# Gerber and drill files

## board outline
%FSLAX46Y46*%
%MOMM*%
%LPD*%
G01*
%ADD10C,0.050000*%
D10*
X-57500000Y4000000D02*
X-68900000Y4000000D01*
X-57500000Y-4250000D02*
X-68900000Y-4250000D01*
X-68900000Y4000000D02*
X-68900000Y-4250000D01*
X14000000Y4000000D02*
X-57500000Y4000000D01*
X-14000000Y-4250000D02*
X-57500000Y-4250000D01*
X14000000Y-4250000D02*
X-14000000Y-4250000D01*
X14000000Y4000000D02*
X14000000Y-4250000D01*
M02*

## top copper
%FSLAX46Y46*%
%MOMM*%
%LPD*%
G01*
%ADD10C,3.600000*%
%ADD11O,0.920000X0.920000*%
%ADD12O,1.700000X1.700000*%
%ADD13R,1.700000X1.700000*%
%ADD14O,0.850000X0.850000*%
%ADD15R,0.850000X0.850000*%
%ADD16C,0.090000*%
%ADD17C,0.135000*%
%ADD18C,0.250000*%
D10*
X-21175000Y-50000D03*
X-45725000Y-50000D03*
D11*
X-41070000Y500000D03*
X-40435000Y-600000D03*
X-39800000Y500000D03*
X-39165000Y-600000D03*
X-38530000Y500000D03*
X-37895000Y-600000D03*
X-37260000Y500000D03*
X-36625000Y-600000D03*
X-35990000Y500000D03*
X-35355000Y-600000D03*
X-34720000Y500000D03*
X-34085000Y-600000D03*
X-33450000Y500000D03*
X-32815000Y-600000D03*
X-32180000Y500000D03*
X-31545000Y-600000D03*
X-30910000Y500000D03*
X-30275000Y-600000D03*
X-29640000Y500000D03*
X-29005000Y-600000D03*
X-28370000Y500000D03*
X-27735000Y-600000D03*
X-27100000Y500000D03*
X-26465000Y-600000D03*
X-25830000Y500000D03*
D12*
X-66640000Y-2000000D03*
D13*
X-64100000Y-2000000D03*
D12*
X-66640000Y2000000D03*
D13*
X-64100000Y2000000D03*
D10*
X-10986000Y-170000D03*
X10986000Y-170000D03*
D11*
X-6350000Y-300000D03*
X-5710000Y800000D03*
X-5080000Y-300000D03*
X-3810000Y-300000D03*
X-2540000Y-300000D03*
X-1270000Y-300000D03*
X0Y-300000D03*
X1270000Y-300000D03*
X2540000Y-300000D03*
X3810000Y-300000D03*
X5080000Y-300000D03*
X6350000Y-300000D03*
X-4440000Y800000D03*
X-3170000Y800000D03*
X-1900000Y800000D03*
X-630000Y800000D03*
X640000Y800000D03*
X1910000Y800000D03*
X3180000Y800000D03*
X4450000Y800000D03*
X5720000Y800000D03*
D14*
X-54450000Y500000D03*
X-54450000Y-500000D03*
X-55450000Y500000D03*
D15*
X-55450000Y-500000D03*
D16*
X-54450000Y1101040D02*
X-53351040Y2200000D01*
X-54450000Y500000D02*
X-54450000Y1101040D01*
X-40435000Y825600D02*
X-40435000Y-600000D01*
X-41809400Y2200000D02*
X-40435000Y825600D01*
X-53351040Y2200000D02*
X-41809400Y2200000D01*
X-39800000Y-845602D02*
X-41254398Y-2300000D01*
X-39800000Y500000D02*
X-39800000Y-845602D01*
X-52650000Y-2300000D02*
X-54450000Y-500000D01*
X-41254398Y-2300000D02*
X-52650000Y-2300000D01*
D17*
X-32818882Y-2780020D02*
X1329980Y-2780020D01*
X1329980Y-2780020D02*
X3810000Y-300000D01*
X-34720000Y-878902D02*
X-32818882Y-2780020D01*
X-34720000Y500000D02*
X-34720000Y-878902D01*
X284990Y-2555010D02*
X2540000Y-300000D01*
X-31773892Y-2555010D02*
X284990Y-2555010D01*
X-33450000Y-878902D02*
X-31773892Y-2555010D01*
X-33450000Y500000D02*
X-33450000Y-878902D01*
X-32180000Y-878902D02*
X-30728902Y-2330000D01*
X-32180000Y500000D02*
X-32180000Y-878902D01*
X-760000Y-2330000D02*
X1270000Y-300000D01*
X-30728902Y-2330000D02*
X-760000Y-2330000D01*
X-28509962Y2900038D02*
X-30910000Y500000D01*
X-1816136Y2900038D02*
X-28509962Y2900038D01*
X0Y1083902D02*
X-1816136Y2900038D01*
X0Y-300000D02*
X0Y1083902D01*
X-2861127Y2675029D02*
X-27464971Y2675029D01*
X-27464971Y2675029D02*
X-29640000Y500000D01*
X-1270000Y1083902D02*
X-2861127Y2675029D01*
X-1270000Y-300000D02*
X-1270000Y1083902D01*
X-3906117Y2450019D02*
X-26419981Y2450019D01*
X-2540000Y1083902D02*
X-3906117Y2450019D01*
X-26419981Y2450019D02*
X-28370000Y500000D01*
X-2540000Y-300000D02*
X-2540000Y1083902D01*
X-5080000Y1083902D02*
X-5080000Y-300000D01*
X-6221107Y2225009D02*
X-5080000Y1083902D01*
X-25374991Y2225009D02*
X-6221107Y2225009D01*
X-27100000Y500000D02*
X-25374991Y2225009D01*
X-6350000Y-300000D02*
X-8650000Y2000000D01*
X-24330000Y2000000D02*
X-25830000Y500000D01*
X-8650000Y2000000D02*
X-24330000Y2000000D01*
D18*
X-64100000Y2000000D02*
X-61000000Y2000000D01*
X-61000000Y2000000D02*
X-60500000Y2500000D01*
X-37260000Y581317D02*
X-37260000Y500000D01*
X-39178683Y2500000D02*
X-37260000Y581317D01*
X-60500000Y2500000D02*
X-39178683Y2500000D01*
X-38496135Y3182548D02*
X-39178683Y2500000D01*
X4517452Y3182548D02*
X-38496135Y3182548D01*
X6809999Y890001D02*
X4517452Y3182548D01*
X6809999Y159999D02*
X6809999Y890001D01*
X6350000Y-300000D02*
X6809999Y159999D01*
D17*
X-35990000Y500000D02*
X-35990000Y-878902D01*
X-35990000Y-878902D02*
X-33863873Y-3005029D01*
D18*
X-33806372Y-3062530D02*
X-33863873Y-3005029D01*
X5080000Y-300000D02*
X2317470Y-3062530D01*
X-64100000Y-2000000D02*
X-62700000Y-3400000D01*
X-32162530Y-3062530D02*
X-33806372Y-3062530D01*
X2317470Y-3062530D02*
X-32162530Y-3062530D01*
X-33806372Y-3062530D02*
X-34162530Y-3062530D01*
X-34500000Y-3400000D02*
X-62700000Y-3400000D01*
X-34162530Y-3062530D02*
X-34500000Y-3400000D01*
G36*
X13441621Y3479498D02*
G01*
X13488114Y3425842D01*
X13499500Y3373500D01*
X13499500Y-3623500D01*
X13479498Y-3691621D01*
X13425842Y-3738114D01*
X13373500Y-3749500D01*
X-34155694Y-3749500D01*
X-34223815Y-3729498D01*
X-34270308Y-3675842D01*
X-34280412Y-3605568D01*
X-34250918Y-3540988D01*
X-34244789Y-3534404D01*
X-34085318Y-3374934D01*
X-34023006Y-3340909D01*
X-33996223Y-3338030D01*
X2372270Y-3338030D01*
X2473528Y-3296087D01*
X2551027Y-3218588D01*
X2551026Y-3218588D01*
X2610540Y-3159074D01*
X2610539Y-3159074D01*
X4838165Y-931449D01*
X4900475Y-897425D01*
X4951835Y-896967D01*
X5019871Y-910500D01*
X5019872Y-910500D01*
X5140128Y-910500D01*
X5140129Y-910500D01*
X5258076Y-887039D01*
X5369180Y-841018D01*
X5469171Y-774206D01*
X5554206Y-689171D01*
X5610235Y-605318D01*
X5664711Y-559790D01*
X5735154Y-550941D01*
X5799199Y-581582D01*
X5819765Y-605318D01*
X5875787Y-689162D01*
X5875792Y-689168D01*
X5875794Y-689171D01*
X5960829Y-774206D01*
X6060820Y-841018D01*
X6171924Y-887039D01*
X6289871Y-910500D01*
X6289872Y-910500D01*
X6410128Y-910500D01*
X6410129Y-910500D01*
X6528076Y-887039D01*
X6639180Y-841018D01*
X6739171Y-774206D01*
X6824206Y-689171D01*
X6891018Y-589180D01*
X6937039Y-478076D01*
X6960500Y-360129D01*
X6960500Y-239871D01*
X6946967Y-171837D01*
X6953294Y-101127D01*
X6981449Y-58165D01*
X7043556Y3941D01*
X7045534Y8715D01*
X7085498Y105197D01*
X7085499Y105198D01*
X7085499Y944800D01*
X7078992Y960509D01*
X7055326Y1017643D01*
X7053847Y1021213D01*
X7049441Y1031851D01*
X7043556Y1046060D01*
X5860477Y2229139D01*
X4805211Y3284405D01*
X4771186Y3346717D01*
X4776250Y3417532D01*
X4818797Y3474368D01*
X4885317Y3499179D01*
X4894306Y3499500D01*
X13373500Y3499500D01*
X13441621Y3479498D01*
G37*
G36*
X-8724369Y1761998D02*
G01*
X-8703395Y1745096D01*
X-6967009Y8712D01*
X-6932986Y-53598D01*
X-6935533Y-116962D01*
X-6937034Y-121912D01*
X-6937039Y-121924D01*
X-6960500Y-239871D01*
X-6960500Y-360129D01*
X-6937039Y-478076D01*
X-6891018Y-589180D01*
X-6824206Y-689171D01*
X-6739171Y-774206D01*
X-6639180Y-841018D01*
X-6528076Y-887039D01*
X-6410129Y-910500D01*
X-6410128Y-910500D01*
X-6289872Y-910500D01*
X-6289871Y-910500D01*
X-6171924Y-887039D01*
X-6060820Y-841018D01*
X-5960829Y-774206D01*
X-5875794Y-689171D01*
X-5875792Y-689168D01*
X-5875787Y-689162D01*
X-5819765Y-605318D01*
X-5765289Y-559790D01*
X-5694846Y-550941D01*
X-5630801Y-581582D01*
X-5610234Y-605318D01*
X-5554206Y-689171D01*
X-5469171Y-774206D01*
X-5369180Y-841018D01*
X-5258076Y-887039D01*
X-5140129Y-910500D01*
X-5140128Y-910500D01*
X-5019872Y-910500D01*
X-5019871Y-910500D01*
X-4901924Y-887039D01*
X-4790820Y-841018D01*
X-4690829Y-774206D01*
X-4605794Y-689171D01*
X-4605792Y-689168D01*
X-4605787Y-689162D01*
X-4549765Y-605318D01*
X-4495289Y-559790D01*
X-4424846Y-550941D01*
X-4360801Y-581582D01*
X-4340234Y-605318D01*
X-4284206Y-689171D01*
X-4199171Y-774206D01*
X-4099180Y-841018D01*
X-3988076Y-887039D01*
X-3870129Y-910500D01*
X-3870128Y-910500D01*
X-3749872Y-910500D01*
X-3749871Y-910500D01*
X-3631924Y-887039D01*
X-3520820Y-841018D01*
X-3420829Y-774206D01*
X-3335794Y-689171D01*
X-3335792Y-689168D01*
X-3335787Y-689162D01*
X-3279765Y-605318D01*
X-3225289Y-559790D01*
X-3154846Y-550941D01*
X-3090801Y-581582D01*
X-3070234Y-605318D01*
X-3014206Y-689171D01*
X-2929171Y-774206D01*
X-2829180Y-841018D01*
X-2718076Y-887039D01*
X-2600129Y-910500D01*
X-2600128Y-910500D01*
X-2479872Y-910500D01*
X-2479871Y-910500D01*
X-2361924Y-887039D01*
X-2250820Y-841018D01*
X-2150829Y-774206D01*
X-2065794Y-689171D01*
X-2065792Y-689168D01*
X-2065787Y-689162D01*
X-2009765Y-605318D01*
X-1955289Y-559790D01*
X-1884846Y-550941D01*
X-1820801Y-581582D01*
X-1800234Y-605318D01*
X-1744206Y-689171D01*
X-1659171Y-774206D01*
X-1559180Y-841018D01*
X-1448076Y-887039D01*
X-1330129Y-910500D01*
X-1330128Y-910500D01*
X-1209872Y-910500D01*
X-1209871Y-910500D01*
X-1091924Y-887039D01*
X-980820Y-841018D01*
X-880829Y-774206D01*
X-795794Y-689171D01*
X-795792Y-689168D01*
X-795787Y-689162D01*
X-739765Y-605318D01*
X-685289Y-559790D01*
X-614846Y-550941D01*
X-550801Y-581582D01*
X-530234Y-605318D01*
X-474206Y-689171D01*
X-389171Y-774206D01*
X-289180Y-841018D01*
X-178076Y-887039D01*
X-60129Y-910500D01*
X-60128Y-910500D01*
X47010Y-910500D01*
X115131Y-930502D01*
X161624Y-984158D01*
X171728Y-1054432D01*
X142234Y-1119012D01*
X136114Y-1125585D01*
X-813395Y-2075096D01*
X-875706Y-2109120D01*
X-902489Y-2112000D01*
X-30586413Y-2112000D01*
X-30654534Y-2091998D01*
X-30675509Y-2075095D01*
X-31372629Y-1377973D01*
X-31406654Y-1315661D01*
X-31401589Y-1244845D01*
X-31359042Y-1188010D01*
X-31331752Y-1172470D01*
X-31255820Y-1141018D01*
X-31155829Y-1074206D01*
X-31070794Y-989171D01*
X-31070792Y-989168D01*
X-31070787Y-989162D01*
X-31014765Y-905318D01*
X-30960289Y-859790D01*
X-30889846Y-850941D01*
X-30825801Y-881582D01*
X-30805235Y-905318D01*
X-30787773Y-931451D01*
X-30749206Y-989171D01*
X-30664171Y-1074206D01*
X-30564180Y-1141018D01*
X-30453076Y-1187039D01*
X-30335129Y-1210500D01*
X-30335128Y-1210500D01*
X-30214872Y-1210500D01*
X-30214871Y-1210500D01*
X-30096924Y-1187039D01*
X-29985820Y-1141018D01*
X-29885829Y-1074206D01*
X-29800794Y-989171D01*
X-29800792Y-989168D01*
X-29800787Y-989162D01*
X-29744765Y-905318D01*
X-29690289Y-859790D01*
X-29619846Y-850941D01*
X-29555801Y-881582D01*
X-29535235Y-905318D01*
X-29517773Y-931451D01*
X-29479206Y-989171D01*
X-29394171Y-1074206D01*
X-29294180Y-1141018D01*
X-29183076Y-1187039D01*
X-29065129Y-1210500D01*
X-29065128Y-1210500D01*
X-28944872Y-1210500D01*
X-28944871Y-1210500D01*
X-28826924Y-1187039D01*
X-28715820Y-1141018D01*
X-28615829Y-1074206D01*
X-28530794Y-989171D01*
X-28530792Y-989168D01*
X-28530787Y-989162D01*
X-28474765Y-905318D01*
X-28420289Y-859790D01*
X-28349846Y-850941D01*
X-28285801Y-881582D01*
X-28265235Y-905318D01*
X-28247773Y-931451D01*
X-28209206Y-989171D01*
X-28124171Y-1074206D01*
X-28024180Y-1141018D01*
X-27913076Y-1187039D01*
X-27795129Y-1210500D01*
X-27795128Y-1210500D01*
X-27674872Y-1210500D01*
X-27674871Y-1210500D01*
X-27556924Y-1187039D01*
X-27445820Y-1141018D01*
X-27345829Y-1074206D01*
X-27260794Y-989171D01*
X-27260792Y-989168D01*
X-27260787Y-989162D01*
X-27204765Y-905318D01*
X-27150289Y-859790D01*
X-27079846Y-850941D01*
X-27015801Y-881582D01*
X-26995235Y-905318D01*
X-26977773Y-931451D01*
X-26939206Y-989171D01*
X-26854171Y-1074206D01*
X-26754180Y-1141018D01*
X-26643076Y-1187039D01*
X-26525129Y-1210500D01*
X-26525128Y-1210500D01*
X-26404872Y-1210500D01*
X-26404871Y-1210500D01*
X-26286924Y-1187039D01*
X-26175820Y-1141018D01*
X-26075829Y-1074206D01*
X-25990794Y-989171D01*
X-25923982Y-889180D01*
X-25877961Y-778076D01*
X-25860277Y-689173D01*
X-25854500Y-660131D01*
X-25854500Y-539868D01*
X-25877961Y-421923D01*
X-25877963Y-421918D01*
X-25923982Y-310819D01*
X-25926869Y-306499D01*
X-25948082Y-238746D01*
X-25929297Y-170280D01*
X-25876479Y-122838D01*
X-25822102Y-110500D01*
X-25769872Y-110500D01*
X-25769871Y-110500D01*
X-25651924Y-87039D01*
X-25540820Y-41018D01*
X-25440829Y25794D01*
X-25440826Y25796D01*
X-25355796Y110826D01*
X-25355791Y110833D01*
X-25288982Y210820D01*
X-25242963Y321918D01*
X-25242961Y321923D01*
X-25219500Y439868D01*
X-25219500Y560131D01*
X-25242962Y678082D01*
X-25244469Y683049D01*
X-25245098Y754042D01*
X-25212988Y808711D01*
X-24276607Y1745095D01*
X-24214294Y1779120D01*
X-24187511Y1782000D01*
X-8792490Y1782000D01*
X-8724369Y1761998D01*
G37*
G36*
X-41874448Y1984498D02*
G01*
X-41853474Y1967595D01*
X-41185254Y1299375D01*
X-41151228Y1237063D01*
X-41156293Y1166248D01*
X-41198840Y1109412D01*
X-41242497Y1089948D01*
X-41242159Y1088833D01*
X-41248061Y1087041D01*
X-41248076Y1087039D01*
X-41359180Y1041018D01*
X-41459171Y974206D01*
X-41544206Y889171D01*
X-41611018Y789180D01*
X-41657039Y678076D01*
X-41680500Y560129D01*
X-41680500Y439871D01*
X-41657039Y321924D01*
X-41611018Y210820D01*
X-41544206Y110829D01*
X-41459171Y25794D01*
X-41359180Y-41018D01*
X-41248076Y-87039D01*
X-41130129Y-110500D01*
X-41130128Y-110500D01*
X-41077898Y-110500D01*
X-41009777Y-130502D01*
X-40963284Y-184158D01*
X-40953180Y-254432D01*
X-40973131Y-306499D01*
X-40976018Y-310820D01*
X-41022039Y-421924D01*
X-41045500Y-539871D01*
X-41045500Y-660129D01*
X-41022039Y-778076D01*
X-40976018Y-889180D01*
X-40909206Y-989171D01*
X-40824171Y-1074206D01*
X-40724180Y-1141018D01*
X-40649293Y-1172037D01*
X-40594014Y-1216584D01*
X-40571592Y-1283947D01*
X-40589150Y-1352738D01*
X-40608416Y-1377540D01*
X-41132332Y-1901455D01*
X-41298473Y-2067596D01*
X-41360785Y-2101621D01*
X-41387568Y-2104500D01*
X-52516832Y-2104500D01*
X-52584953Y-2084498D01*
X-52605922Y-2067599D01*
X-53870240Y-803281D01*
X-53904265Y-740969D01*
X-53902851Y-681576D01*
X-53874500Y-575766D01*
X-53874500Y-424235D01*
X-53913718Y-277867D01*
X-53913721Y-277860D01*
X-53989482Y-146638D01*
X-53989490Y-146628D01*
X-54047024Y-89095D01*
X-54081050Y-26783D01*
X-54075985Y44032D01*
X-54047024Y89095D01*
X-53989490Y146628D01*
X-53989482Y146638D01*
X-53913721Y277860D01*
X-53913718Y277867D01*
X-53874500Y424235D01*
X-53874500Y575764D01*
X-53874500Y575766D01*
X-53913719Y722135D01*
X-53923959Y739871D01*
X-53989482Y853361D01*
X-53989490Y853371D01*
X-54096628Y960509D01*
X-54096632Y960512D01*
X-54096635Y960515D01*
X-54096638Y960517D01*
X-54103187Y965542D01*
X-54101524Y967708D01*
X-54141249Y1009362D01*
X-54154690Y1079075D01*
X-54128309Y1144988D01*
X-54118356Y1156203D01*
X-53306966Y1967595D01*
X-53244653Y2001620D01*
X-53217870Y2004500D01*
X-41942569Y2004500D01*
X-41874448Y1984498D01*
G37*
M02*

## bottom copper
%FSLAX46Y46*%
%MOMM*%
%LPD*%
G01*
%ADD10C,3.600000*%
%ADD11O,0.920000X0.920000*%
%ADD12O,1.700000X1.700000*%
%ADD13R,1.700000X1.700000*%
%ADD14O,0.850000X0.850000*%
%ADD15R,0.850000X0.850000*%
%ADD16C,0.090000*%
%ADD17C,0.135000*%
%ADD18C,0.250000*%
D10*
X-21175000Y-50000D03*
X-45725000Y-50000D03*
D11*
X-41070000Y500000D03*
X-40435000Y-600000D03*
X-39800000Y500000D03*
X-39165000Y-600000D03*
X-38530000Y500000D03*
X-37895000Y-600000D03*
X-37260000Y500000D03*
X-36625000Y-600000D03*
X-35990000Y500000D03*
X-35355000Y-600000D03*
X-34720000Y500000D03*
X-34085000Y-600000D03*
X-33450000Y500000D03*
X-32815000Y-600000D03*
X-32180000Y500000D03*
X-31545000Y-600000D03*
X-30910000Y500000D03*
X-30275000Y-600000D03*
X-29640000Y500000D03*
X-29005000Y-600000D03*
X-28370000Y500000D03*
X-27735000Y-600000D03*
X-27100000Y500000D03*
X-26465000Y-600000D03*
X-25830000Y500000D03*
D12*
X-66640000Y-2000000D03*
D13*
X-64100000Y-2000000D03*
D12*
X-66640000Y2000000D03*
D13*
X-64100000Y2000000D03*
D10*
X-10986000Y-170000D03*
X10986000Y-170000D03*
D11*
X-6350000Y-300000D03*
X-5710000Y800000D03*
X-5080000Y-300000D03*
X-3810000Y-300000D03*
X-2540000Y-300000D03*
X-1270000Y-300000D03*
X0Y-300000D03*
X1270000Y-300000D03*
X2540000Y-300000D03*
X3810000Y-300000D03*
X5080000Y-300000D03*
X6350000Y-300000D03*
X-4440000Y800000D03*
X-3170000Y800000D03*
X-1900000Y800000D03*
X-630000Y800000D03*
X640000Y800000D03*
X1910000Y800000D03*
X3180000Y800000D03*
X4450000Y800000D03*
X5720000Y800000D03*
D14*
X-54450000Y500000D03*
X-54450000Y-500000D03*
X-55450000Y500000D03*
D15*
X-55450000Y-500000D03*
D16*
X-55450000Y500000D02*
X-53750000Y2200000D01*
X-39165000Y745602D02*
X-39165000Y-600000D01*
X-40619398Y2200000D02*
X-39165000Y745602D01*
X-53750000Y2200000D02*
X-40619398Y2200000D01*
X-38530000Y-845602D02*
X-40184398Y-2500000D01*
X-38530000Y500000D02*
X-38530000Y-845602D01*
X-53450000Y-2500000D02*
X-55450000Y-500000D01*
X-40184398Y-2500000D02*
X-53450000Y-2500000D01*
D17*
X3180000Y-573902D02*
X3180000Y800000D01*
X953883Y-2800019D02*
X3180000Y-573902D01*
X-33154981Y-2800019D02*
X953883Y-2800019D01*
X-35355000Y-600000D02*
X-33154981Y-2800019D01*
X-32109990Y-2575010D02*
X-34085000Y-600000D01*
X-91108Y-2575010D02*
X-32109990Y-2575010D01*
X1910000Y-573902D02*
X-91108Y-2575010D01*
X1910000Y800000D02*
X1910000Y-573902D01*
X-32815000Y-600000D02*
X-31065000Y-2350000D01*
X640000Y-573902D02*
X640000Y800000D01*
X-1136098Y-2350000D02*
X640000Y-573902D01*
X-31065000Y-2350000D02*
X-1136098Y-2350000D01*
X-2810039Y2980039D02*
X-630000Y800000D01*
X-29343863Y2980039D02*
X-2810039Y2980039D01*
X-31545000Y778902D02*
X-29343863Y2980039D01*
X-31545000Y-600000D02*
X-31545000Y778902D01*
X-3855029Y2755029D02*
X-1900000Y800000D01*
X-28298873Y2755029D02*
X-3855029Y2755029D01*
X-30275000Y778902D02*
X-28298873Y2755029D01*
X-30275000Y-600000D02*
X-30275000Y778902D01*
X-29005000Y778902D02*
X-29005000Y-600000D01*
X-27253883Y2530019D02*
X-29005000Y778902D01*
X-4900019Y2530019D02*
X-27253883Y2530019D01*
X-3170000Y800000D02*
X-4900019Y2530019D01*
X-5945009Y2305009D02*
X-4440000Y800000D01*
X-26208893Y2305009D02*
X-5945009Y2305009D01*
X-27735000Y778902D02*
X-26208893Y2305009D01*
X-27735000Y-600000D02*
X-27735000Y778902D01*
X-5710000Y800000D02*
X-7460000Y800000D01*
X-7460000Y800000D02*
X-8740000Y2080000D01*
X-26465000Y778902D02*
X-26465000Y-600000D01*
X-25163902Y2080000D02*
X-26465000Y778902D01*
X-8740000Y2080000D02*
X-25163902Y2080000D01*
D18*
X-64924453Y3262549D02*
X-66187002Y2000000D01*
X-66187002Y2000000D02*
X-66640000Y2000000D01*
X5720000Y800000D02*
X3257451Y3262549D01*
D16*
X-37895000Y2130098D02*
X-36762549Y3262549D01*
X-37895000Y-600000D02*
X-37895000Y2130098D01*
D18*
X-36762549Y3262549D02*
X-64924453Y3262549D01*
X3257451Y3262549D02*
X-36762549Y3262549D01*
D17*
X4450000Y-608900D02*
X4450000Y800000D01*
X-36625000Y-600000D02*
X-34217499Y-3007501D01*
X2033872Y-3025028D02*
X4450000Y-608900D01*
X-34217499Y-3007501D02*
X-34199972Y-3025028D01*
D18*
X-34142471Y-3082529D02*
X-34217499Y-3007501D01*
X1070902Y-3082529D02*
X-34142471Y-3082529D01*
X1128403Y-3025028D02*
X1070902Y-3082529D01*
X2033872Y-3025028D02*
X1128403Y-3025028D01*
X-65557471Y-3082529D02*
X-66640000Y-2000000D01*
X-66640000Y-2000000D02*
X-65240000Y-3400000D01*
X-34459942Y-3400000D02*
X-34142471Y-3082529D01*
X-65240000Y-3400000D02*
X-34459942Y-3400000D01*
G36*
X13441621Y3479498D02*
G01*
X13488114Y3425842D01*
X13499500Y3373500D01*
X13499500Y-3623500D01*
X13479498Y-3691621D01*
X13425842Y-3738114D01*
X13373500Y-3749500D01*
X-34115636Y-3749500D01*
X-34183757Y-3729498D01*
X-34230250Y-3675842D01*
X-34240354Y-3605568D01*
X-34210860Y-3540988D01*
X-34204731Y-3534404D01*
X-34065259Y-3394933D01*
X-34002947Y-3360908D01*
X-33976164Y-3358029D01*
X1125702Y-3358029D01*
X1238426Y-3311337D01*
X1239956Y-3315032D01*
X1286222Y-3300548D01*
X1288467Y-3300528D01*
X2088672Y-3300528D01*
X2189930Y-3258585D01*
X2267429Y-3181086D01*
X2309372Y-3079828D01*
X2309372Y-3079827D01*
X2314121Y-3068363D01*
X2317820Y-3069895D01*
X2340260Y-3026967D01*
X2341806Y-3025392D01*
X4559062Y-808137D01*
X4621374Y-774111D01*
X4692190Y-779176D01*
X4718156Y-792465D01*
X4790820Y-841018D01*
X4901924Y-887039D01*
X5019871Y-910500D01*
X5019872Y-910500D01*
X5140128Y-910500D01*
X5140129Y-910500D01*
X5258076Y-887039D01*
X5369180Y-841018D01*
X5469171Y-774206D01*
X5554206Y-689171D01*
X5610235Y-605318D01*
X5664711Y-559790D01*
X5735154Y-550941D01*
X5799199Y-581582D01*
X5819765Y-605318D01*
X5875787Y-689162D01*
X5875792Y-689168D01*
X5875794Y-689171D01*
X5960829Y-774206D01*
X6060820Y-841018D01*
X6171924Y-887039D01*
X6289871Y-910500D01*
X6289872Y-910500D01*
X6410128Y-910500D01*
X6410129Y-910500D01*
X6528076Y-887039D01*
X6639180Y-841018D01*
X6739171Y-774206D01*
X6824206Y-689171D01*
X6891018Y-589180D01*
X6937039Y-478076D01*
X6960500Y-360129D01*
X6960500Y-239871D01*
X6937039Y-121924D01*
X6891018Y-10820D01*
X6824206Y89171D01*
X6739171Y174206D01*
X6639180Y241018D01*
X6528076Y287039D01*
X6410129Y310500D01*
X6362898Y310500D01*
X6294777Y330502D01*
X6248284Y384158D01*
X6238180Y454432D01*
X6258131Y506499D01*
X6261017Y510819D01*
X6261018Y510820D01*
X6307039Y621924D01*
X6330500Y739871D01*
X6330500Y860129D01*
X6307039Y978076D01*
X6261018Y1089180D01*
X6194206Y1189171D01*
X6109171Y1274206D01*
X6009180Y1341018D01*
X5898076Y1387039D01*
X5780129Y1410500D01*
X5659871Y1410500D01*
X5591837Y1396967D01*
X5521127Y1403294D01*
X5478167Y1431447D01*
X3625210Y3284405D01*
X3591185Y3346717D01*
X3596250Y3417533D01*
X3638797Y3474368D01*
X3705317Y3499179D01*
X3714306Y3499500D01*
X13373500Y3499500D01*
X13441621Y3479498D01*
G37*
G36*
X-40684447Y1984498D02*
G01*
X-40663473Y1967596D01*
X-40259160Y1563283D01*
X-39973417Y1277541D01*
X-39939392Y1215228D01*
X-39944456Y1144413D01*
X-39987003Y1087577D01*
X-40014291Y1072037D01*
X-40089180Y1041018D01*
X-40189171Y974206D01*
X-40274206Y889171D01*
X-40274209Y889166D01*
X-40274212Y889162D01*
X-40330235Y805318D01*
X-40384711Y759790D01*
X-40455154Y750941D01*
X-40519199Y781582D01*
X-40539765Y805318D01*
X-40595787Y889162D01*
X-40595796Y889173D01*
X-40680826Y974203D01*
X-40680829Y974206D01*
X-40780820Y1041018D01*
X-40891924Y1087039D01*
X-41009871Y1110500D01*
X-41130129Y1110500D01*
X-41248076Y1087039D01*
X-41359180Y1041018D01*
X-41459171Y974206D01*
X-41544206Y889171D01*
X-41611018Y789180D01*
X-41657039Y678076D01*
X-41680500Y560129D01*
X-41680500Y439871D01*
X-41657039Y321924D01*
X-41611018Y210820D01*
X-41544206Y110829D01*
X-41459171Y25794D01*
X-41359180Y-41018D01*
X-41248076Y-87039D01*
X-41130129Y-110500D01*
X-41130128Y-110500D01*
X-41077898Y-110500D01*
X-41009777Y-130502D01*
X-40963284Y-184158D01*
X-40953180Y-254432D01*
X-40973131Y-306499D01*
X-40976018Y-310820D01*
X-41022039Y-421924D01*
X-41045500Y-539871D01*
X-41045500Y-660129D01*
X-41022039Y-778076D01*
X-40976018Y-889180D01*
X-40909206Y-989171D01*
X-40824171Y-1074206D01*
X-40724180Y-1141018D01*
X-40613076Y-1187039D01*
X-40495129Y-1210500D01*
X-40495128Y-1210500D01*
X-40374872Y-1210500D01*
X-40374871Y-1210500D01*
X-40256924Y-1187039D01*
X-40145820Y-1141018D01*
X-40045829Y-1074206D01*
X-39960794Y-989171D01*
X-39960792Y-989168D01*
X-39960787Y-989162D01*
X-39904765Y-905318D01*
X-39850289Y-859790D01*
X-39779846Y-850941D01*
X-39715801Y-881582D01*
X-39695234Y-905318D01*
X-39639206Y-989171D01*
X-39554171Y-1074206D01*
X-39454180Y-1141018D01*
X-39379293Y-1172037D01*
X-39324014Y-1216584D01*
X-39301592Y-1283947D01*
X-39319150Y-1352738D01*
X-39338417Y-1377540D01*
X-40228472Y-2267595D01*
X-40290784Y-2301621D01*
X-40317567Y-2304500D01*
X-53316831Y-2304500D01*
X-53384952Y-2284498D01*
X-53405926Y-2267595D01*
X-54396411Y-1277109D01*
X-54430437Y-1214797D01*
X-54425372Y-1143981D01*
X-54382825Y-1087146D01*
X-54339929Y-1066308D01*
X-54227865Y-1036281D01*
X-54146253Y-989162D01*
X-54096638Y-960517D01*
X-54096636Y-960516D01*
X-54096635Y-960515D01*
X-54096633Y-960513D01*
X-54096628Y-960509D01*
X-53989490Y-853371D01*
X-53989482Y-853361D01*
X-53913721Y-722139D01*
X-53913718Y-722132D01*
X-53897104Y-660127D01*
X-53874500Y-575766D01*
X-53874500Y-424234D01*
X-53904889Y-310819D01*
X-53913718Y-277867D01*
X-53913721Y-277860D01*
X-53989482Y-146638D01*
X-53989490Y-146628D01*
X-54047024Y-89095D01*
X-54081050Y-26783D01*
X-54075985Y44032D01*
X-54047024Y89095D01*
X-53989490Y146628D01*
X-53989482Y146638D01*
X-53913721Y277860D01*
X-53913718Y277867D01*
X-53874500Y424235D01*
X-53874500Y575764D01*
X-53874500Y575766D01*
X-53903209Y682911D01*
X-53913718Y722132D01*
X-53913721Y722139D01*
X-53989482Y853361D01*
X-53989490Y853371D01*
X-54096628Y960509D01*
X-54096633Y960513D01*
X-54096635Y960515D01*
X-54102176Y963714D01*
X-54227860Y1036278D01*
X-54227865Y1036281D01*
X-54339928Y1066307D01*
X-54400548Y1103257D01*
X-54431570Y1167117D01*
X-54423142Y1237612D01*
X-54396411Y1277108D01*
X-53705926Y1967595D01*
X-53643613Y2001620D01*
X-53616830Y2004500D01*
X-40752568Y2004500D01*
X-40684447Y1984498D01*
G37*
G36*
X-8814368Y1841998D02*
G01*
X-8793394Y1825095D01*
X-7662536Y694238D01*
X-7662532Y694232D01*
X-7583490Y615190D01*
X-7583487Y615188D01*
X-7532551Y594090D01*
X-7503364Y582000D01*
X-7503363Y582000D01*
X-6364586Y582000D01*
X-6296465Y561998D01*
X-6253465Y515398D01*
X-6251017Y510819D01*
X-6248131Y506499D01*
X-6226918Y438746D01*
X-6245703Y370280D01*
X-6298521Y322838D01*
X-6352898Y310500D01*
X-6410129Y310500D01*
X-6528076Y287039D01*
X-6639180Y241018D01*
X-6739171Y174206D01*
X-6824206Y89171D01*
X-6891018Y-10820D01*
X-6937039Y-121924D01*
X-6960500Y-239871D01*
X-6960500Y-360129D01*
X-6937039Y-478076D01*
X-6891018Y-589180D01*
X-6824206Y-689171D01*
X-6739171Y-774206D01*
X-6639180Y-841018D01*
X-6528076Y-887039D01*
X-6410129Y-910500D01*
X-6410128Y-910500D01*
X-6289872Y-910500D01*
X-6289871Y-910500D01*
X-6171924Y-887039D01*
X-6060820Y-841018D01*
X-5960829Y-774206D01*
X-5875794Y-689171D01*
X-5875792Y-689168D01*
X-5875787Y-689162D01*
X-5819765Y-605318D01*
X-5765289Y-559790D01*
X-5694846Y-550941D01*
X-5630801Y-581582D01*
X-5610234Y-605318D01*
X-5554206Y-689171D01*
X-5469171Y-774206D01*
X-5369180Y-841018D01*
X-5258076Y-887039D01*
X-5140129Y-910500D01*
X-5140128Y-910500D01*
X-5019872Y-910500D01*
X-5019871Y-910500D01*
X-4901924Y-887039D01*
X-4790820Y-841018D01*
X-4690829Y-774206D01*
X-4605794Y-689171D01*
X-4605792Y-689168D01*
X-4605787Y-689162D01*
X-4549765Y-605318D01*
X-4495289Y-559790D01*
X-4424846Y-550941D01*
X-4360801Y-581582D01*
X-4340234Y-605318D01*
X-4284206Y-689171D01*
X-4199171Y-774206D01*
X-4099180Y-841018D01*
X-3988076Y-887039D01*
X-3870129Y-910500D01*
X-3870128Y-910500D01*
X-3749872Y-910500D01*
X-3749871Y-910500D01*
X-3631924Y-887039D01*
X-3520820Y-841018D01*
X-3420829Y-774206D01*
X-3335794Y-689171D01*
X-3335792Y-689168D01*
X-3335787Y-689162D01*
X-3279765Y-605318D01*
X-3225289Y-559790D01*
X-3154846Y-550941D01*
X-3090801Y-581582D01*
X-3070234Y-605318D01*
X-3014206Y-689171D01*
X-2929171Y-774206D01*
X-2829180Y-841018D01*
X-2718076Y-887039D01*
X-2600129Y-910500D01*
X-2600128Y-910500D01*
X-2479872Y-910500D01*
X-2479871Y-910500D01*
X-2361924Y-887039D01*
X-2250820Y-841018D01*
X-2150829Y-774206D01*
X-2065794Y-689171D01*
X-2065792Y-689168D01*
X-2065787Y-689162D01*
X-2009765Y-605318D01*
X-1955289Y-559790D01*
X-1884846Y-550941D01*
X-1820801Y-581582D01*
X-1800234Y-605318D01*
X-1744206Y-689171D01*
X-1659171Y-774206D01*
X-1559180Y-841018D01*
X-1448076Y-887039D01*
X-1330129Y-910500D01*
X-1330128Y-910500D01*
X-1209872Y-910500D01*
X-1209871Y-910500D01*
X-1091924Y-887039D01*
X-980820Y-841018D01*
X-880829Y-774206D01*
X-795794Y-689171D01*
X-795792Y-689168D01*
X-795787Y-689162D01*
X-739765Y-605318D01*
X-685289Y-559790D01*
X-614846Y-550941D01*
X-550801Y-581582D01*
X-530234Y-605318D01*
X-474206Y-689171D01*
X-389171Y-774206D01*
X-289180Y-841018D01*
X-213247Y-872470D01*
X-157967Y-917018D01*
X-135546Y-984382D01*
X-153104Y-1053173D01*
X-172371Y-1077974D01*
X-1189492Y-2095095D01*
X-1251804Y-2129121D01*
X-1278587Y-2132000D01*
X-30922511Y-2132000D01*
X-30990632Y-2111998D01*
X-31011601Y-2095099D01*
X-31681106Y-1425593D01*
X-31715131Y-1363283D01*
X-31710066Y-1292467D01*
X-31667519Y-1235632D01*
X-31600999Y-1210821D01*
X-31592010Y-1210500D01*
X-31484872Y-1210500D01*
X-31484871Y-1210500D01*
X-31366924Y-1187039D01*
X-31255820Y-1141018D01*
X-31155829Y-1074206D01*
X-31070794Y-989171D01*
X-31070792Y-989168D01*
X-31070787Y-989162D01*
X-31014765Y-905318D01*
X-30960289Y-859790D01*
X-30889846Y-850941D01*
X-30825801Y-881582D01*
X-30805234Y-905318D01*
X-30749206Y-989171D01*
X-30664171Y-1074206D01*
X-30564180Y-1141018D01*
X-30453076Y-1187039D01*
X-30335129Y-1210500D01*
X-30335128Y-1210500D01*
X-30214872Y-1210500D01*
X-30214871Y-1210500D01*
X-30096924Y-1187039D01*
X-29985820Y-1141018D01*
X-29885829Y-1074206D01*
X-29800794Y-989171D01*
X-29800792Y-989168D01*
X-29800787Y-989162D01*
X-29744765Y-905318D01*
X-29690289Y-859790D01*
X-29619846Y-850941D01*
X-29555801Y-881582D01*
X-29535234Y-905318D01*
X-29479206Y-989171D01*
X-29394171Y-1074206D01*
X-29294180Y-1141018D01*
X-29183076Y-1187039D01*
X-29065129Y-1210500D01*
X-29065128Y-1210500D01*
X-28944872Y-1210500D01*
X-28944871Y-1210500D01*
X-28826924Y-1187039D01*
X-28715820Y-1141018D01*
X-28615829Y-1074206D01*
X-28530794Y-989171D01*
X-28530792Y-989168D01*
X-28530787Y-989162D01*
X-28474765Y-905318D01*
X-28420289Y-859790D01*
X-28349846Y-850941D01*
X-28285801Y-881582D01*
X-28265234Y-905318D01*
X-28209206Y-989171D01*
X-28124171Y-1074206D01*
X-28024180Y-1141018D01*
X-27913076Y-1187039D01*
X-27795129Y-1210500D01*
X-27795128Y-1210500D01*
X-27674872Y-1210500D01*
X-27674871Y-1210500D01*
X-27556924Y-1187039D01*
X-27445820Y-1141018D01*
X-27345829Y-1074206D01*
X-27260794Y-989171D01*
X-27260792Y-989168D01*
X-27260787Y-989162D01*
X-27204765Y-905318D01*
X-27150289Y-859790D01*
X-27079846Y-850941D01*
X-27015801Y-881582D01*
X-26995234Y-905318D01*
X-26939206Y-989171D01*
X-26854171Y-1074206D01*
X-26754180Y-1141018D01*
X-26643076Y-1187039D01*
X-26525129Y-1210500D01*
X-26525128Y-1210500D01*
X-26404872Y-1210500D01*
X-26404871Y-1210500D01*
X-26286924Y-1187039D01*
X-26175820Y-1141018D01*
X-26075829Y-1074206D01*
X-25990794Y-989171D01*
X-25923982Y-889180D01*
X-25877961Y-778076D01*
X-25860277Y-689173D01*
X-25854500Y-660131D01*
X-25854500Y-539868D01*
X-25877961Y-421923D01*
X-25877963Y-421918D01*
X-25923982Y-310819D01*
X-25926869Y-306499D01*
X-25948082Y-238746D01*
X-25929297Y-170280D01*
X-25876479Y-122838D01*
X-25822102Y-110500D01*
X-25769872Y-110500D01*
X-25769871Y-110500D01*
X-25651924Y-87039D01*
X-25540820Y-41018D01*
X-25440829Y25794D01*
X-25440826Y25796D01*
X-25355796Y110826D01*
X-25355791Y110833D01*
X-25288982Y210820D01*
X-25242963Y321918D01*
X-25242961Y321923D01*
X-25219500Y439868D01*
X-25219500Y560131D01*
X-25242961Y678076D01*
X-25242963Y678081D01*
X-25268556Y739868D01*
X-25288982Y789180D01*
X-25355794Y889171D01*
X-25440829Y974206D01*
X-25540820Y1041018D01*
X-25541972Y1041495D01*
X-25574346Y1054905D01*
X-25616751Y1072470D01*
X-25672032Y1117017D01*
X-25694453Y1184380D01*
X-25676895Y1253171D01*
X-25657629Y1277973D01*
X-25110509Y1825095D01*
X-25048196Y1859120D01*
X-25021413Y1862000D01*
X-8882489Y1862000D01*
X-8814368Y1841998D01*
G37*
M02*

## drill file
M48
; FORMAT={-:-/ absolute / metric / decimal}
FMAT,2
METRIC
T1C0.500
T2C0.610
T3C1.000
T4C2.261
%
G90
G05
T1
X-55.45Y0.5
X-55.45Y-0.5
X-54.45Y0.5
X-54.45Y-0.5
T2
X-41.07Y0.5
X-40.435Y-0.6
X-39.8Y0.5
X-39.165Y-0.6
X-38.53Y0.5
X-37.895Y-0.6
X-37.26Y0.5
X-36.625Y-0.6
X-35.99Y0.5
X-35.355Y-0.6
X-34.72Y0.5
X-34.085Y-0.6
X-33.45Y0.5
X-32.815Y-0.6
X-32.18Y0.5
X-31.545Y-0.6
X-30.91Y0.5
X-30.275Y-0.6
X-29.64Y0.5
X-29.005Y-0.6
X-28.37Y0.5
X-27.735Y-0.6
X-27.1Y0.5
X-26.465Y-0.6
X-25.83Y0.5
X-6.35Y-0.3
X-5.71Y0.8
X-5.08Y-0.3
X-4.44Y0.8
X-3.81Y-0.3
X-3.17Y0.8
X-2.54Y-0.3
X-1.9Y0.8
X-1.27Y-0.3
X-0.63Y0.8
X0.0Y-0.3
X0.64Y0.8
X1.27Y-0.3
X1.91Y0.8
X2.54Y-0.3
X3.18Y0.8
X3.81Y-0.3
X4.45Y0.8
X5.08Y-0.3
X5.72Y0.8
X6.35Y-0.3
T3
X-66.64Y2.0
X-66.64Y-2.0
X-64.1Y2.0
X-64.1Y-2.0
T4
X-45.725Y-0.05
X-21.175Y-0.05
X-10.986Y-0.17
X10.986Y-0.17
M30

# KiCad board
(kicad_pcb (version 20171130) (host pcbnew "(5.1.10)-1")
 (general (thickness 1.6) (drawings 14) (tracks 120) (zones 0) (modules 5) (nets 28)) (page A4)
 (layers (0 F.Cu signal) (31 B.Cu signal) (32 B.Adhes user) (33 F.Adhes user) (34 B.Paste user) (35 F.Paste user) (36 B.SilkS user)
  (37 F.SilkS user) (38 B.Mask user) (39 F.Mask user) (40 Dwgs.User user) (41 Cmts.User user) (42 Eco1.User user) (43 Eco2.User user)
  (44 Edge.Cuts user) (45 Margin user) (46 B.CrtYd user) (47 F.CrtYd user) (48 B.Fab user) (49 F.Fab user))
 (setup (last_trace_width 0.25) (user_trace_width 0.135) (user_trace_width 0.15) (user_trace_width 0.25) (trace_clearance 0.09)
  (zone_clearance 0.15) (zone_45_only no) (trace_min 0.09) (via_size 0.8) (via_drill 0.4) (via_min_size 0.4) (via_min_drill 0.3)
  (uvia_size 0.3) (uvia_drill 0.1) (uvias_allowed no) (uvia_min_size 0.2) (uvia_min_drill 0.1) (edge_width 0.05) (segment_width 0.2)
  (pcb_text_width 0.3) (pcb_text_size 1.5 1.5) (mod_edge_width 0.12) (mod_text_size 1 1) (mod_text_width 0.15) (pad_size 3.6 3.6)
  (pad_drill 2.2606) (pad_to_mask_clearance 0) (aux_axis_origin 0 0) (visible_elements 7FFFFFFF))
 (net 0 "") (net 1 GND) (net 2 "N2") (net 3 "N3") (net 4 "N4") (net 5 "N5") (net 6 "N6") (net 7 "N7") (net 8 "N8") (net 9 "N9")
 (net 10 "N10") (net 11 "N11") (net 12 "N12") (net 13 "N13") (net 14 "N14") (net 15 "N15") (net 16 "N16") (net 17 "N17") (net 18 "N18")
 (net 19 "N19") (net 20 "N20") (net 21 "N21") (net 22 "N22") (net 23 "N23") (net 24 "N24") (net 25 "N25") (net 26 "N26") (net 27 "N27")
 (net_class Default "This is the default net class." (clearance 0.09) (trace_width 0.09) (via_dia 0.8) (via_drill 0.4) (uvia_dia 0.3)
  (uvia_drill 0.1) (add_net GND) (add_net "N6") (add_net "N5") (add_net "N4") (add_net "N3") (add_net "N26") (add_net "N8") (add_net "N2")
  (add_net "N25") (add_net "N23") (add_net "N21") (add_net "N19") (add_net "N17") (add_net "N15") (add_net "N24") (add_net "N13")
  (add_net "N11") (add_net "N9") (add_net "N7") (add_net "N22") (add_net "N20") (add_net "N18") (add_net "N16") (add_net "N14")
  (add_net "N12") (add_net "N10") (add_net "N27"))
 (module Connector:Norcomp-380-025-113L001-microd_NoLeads (layer B.Cu) (at -33.45 0.05 180)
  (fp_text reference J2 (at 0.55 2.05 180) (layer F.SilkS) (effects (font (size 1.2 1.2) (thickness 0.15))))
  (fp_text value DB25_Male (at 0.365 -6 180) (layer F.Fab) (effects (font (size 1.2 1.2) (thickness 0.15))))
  (pad 0 thru_hole circle (at -12.275 0 180) (size 3.6 3.6) (drill 2.2606) (layers *.Cu *.Mask) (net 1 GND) (zone_connect 2))
  (pad 0 thru_hole circle (at 12.275 0 180) (size 3.6 3.6) (drill 2.2606) (layers *.Cu *.Mask) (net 1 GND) (zone_connect 2))
  (pad 13 thru_hole oval (at 7.62 0.55 180) (size 0.92 0.92) (drill 0.61) (layers *.Cu *.Mask) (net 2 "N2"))
  (pad 25 thru_hole oval (at 6.985 -0.55 180) (size 0.92 0.92) (drill 0.61) (layers *.Cu *.Mask) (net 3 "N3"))
  (pad 12 thru_hole oval (at 6.35 0.55 180) (size 0.92 0.92) (drill 0.61) (layers *.Cu *.Mask) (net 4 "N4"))
  (pad 24 thru_hole oval (at 5.715 -0.55 180) (size 0.92 0.92) (drill 0.61) (layers *.Cu *.Mask) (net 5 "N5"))
  (pad 11 thru_hole oval (at 5.08 0.55 180) (size 0.92 0.92) (drill 0.61) (layers *.Cu *.Mask) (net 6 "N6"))
  (pad 23 thru_hole oval (at 4.445 -0.55 180) (size 0.92 0.92) (drill 0.61) (layers *.Cu *.Mask) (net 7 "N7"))
  (pad 10 thru_hole oval (at 3.81 0.55 180) (size 0.92 0.92) (drill 0.61) (layers *.Cu *.Mask) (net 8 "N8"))
  (pad 22 thru_hole oval (at 3.175 -0.55 180) (size 0.92 0.92) (drill 0.61) (layers *.Cu *.Mask) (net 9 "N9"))
  (pad 9 thru_hole oval (at 2.54 0.55 180) (size 0.92 0.92) (drill 0.61) (layers *.Cu *.Mask) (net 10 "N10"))
  (pad 21 thru_hole oval (at 1.905 -0.55 180) (size 0.92 0.92) (drill 0.61) (layers *.Cu *.Mask) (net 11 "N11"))
  (pad 8 thru_hole oval (at 1.27 0.55 180) (size 0.92 0.92) (drill 0.61) (layers *.Cu *.Mask) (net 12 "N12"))
  (pad 20 thru_hole oval (at 0.635 -0.55 180) (size 0.92 0.92) (drill 0.61) (layers *.Cu *.Mask) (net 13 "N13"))
  (pad 7 thru_hole oval (at 0 0.55 180) (size 0.92 0.92) (drill 0.61) (layers *.Cu *.Mask) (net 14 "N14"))
  (pad 19 thru_hole oval (at -0.635 -0.55 180) (size 0.92 0.92) (drill 0.61) (layers *.Cu *.Mask) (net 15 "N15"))
  (pad 6 thru_hole oval (at -1.27 0.55 180) (size 0.92 0.92) (drill 0.61) (layers *.Cu *.Mask) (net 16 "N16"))
  (pad 18 thru_hole oval (at -1.905 -0.55 180) (size 0.92 0.92) (drill 0.61) (layers *.Cu *.Mask) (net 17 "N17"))
  (pad 5 thru_hole oval (at -2.54 0.55 180) (size 0.92 0.92) (drill 0.61) (layers *.Cu *.Mask) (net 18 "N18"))
  (pad 17 thru_hole oval (at -3.175 -0.55 180) (size 0.92 0.92) (drill 0.61) (layers *.Cu *.Mask) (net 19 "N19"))
  (pad 4 thru_hole oval (at -3.81 0.55 180) (size 0.92 0.92) (drill 0.61) (layers *.Cu *.Mask) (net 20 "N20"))
  (pad 16 thru_hole oval (at -4.445 -0.55 180) (size 0.92 0.92) (drill 0.61) (layers *.Cu *.Mask) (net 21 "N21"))
  (pad 3 thru_hole oval (at -5.08 0.55 180) (size 0.92 0.92) (drill 0.61) (layers *.Cu *.Mask) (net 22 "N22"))
  (pad 15 thru_hole oval (at -5.715 -0.55 180) (size 0.92 0.92) (drill 0.61) (layers *.Cu *.Mask) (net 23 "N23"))
  (pad 2 thru_hole oval (at -6.35 0.55 180) (size 0.92 0.92) (drill 0.61) (layers *.Cu *.Mask) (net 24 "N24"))
  (pad 14 thru_hole oval (at -6.985 -0.55 180) (size 0.92 0.92) (drill 0.61) (layers *.Cu *.Mask) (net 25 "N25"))
  (pad 1 thru_hole oval (at -7.62 0.55 180) (size 0.92 0.92) (drill 0.61) (layers *.Cu *.Mask) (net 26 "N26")))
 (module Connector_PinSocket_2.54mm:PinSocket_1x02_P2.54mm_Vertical (layer F.Cu) (at -64.1 2 270)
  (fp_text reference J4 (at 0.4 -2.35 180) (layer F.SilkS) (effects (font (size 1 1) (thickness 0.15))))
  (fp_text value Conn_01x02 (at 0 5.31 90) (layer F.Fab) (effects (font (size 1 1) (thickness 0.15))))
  (pad 2 thru_hole oval (at 0 2.54 270) (size 1.7 1.7) (drill 1) (layers *.Cu *.Mask) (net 9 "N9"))
  (pad 1 thru_hole rect (at 0 0 270) (size 1.7 1.7) (drill 1) (layers *.Cu *.Mask) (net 10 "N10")))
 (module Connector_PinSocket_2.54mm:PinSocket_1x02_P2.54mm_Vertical (layer F.Cu) (at -64.1 -2 270)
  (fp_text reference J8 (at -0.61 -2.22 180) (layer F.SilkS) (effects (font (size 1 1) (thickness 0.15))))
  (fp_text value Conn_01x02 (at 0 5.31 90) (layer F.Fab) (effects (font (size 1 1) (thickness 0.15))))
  (pad 2 thru_hole oval (at 0 2.54 270) (size 1.7 1.7) (drill 1) (layers *.Cu *.Mask) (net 7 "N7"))
  (pad 1 thru_hole rect (at 0 0 270) (size 1.7 1.7) (drill 1) (layers *.Cu *.Mask) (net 8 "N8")))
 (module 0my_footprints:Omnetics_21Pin (layer B.Cu) (at -6.35 0.17 180)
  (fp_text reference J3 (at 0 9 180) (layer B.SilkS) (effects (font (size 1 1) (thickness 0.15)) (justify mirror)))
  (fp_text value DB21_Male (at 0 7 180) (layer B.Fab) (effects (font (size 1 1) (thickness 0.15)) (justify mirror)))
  (pad 0 thru_hole circle (at 4.636 0 180) (size 3.6 3.6) (drill 2.2606) (layers *.Cu *.Mask) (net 1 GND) (zone_connect 2))
  (pad 0 thru_hole circle (at -17.336 0 180) (size 3.6 3.6) (drill 2.2606) (layers *.Cu *.Mask Dwgs.User) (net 1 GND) (zone_connect 2))
  (pad 1 thru_hole oval (at 0 -0.13 180) (size 0.92 0.92) (drill 0.61) (layers *.Cu *.Mask) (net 26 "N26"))
  (pad 12 thru_hole oval (at -0.64 0.97 180) (size 0.92 0.92) (drill 0.61) (layers *.Cu *.Mask) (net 25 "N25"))
  (pad 2 thru_hole oval (at -1.27 -0.13 180) (size 0.92 0.92) (drill 0.61) (layers *.Cu *.Mask) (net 24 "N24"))
  (pad 3 thru_hole oval (at -2.54 -0.13 180) (size 0.92 0.92) (drill 0.61) (layers *.Cu *.Mask) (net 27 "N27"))
  (pad 4 thru_hole oval (at -3.81 -0.13 180) (size 0.92 0.92) (drill 0.61) (layers *.Cu *.Mask) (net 22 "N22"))
  (pad 5 thru_hole oval (at -5.08 -0.13 180) (size 0.92 0.92) (drill 0.61) (layers *.Cu *.Mask) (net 20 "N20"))
  (pad 6 thru_hole oval (at -6.35 -0.13 180) (size 0.92 0.92) (drill 0.61) (layers *.Cu *.Mask) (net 18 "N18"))
  (pad 7 thru_hole oval (at -7.62 -0.13 180) (size 0.92 0.92) (drill 0.61) (layers *.Cu *.Mask) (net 16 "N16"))
  (pad 8 thru_hole oval (at -8.89 -0.13 180) (size 0.92 0.92) (drill 0.61) (layers *.Cu *.Mask) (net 14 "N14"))
  (pad 9 thru_hole oval (at -10.16 -0.13 180) (size 0.92 0.92) (drill 0.61) (layers *.Cu *.Mask) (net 12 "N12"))
  (pad 10 thru_hole oval (at -11.43 -0.13 180) (size 0.92 0.92) (drill 0.61) (layers *.Cu *.Mask) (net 10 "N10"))
  (pad 11 thru_hole oval (at -12.7 -0.13 180) (size 0.92 0.92) (drill 0.61) (layers *.Cu *.Mask) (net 8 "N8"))
  (pad 13 thru_hole oval (at -1.91 0.97 180) (size 0.92 0.92) (drill 0.61) (layers *.Cu *.Mask) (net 23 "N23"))
  (pad 14 thru_hole oval (at -3.18 0.97 180) (size 0.92 0.92) (drill 0.61) (layers *.Cu *.Mask) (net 21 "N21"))
  (pad 15 thru_hole oval (at -4.45 0.97 180) (size 0.92 0.92) (drill 0.61) (layers *.Cu *.Mask) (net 19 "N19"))
  (pad 16 thru_hole oval (at -5.72 0.97 180) (size 0.92 0.92) (drill 0.61) (layers *.Cu *.Mask) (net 17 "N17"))
  (pad 17 thru_hole oval (at -6.99 0.97 180) (size 0.92 0.92) (drill 0.61) (layers *.Cu *.Mask) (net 15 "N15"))
  (pad 18 thru_hole oval (at -8.26 0.97 180) (size 0.92 0.92) (drill 0.61) (layers *.Cu *.Mask) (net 13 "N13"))
  (pad 19 thru_hole oval (at -9.53 0.97 180) (size 0.92 0.92) (drill 0.61) (layers *.Cu *.Mask) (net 11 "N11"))
  (pad 20 thru_hole oval (at -10.8 0.97 180) (size 0.92 0.92) (drill 0.61) (layers *.Cu *.Mask) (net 9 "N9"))
  (pad 21 thru_hole oval (at -12.07 0.97 180) (size 0.92 0.92) (drill 0.61) (layers *.Cu *.Mask) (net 7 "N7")))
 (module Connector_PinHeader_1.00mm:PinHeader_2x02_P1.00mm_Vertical (layer F.Cu) (at -55.45 0.5 90)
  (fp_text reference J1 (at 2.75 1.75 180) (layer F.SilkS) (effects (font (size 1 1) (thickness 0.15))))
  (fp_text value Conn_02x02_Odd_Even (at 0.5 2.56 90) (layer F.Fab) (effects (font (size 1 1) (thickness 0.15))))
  (pad 4 thru_hole oval (at 1 1 90) (size 0.85 0.85) (drill 0.5) (layers *.Cu *.Mask) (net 3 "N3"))
  (pad 3 thru_hole oval (at 0 1 90) (size 0.85 0.85) (drill 0.5) (layers *.Cu *.Mask) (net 4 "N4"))
  (pad 2 thru_hole oval (at 1 0 90) (size 0.85 0.85) (drill 0.5) (layers *.Cu *.Mask) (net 5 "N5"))
  (pad 1 thru_hole rect (at 0 0 90) (size 0.85 0.85) (drill 0.5) (layers *.Cu *.Mask) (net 6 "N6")))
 (gr_line (start -57.5 -4) (end -68.9 -4) (layer Edge.Cuts) (width 0.05))
 (gr_line (start -57.5 4.25) (end -68.9 4.25) (layer Edge.Cuts) (width 0.05))
 (gr_line (start -68.9 -4) (end -68.9 4.25) (layer Edge.Cuts) (width 0.05))
 (gr_line (start 14 -4) (end -57.5 -4) (layer Edge.Cuts) (width 0.05))
 (gr_line (start -14 4.25) (end -57.5 4.25) (layer Edge.Cuts) (width 0.05))
 (gr_line (start 14 4.25) (end -14 4.25) (layer Edge.Cuts) (width 0.05))
 (gr_line (start 14 -4) (end 14 4.25) (layer Edge.Cuts) (width 0.05))
 (segment (start -54.45 -1.10104) (end -53.35104 -2.2) (width 0.09) (layer F.Cu) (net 3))
 (segment (start -54.45 -0.5) (end -54.45 -1.10104) (width 0.09) (layer F.Cu) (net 3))
 (segment (start -40.435 -0.8256) (end -40.435 0.6) (width 0.09) (layer F.Cu) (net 3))
 (segment (start -41.8094 -2.2) (end -40.435 -0.8256) (width 0.09) (layer F.Cu) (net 3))
 (segment (start -53.35104 -2.2) (end -41.8094 -2.2) (width 0.09) (layer F.Cu) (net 3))
 (segment (start -39.8 0.845602) (end -41.254398 2.3) (width 0.09) (layer F.Cu) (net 4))
 (segment (start -39.8 -0.5) (end -39.8 0.845602) (width 0.09) (layer F.Cu) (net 4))
 (segment (start -52.65 2.3) (end -54.45 0.5) (width 0.09) (layer F.Cu) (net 4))
 (segment (start -41.254398 2.3) (end -52.65 2.3) (width 0.09) (layer F.Cu) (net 4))
 (segment (start -55.45 -0.5) (end -53.75 -2.2) (width 0.09) (layer B.Cu) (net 5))
 (segment (start -39.165 -0.745602) (end -39.165 0.6) (width 0.09) (layer B.Cu) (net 5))
 (segment (start -40.619398 -2.2) (end -39.165 -0.745602) (width 0.09) (layer B.Cu) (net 5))
 (segment (start -53.75 -2.2) (end -40.619398 -2.2) (width 0.09) (layer B.Cu) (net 5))
 (segment (start -38.53 0.845602) (end -40.184398 2.5) (width 0.09) (layer B.Cu) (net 6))
 (segment (start -38.53 -0.5) (end -38.53 0.845602) (width 0.09) (layer B.Cu) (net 6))
 (segment (start -53.45 2.5) (end -55.45 0.5) (width 0.09) (layer B.Cu) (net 6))
 (segment (start -40.184398 2.5) (end -53.45 2.5) (width 0.09) (layer B.Cu) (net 6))
 (segment (start 3.18 0.573902) (end 3.18 -0.8) (width 0.135) (layer B.Cu) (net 11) (status 20))
 (segment (start 0.953883 2.800019) (end 3.18 0.573902) (width 0.135) (layer B.Cu) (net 11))
 (segment (start -33.154981 2.800019) (end 0.953883 2.800019) (width 0.135) (layer B.Cu) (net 11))
 (segment (start -35.355 0.6) (end -33.154981 2.800019) (width 0.135) (layer B.Cu) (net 11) (status 10))
 (segment (start -32.818882 2.78002) (end 1.32998 2.78002) (width 0.135) (layer F.Cu) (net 12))
 (segment (start 1.32998 2.78002) (end 3.81 0.3) (width 0.135) (layer F.Cu) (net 12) (status 20))
 (segment (start -34.72 0.878902) (end -32.818882 2.78002) (width 0.135) (layer F.Cu) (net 12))
 (segment (start -34.72 -0.5) (end -34.72 0.878902) (width 0.135) (layer F.Cu) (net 12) (status 10))
 (segment (start -32.10999 2.57501) (end -34.085 0.6) (width 0.135) (layer B.Cu) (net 13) (status 20))
 (segment (start -0.091108 2.57501) (end -32.10999 2.57501) (width 0.135) (layer B.Cu) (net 13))
 (segment (start 1.91 0.573902) (end -0.091108 2.57501) (width 0.135) (layer B.Cu) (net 13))
 (segment (start 1.91 -0.8) (end 1.91 0.573902) (width 0.135) (layer B.Cu) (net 13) (status 10))
 (segment (start 0.28499 2.55501) (end 2.54 0.3) (width 0.135) (layer F.Cu) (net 14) (status 20))
 (segment (start -31.773892 2.55501) (end 0.28499 2.55501) (width 0.135) (layer F.Cu) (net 14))
 (segment (start -33.45 0.878902) (end -31.773892 2.55501) (width 0.135) (layer F.Cu) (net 14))
 (segment (start -33.45 -0.5) (end -33.45 0.878902) (width 0.135) (layer F.Cu) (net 14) (status 10))
 (segment (start -32.815 0.6) (end -31.065 2.35) (width 0.135) (layer B.Cu) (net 15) (status 10))
 (segment (start 0.64 0.573902) (end 0.64 -0.8) (width 0.135) (layer B.Cu) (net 15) (status 20))
 (segment (start -1.136098 2.35) (end 0.64 0.573902) (width 0.135) (layer B.Cu) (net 15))
 (segment (start -31.065 2.35) (end -1.136098 2.35) (width 0.135) (layer B.Cu) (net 15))
 (segment (start -32.18 0.878902) (end -30.728902 2.33) (width 0.135) (layer F.Cu) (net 16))
 (segment (start -32.18 -0.5) (end -32.18 0.878902) (width 0.135) (layer F.Cu) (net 16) (status 10))
 (segment (start -0.76 2.33) (end 1.27 0.3) (width 0.135) (layer F.Cu) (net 16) (status 20))
 (segment (start -30.728902 2.33) (end -0.76 2.33) (width 0.135) (layer F.Cu) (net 16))
 (segment (start -2.810039 -2.980039) (end -0.63 -0.8) (width 0.135) (layer B.Cu) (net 17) (status 20))
 (segment (start -29.343863 -2.980039) (end -2.810039 -2.980039) (width 0.135) (layer B.Cu) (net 17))
 (segment (start -31.545 -0.778902) (end -29.343863 -2.980039) (width 0.135) (layer B.Cu) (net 17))
 (segment (start -31.545 0.6) (end -31.545 -0.778902) (width 0.135) (layer B.Cu) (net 17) (status 10))
 (segment (start -28.509962 -2.900038) (end -30.91 -0.5) (width 0.135) (layer F.Cu) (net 18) (status 20))
 (segment (start -1.816136 -2.900038) (end -28.509962 -2.900038) (width 0.135) (layer F.Cu) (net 18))
 (segment (start 0 -1.083902) (end -1.816136 -2.900038) (width 0.135) (layer F.Cu) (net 18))
 (segment (start 0 0.3) (end 0 -1.083902) (width 0.135) (layer F.Cu) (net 18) (status 10))
 (segment (start -3.855029 -2.755029) (end -1.9 -0.8) (width 0.135) (layer B.Cu) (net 19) (status 20))
 (segment (start -28.298873 -2.755029) (end -3.855029 -2.755029) (width 0.135) (layer B.Cu) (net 19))
 (segment (start -30.275 -0.778902) (end -28.298873 -2.755029) (width 0.135) (layer B.Cu) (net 19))
 (segment (start -30.275 0.6) (end -30.275 -0.778902) (width 0.135) (layer B.Cu) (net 19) (status 10))
 (segment (start -2.861127 -2.675029) (end -27.464971 -2.675029) (width 0.135) (layer F.Cu) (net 20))
 (segment (start -27.464971 -2.675029) (end -29.64 -0.5) (width 0.135) (layer F.Cu) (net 20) (status 20))
 (segment (start -1.27 -1.083902) (end -2.861127 -2.675029) (width 0.135) (layer F.Cu) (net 20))
 (segment (start -1.27 0.3) (end -1.27 -1.083902) (width 0.135) (layer F.Cu) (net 20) (status 10))
 (segment (start -29.005 -0.778902) (end -29.005 0.6) (width 0.135) (layer B.Cu) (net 21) (status 20))
 (segment (start -27.253883 -2.530019) (end -29.005 -0.778902) (width 0.135) (layer B.Cu) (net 21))
 (segment (start -4.900019 -2.530019) (end -27.253883 -2.530019) (width 0.135) (layer B.Cu) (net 21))
 (segment (start -3.17 -0.8) (end -4.900019 -2.530019) (width 0.135) (layer B.Cu) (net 21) (status 10))
 (segment (start -3.906117 -2.450019) (end -26.419981 -2.450019) (width 0.135) (layer F.Cu) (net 22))
 (segment (start -2.54 -1.083902) (end -3.906117 -2.450019) (width 0.135) (layer F.Cu) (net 22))
 (segment (start -26.419981 -2.450019) (end -28.37 -0.5) (width 0.135) (layer F.Cu) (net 22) (status 20))
 (segment (start -2.54 0.3) (end -2.54 -1.083902) (width 0.135) (layer F.Cu) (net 22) (status 10))
 (segment (start -5.945009 -2.305009) (end -4.44 -0.8) (width 0.135) (layer B.Cu) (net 23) (status 20))
 (segment (start -26.208893 -2.305009) (end -5.945009 -2.305009) (width 0.135) (layer B.Cu) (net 23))
 (segment (start -27.735 -0.778902) (end -26.208893 -2.305009) (width 0.135) (layer B.Cu) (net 23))
 (segment (start -27.735 0.6) (end -27.735 -0.778902) (width 0.135) (layer B.Cu) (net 23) (status 10))
 (segment (start -5.08 -1.083902) (end -5.08 0.3) (width 0.135) (layer F.Cu) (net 24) (status 20))
 (segment (start -6.221107 -2.225009) (end -5.08 -1.083902) (width 0.135) (layer F.Cu) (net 24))
 (segment (start -25.374991 -2.225009) (end -6.221107 -2.225009) (width 0.135) (layer F.Cu) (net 24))
 (segment (start -27.1 -0.5) (end -25.374991 -2.225009) (width 0.135) (layer F.Cu) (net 24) (status 10))
 (segment (start -5.71 -0.8) (end -7.46 -0.8) (width 0.135) (layer B.Cu) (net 25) (status 10))
 (segment (start -7.46 -0.8) (end -8.74 -2.08) (width 0.135) (layer B.Cu) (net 25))
 (segment (start -26.465 -0.778902) (end -26.465 0.6) (width 0.135) (layer B.Cu) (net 25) (status 20))
 (segment (start -25.163902 -2.08) (end -26.465 -0.778902) (width 0.135) (layer B.Cu) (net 25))
 (segment (start -8.74 -2.08) (end -25.163902 -2.08) (width 0.135) (layer B.Cu) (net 25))
 (segment (start -6.35 0.3) (end -8.65 -2) (width 0.135) (layer F.Cu) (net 26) (status 10))
 (segment (start -24.33 -2) (end -25.83 -0.5) (width 0.135) (layer F.Cu) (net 26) (status 20))
 (segment (start -8.65 -2) (end -24.33 -2) (width 0.135) (layer F.Cu) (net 26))
 (segment (start -64.924453 -3.262549) (end -66.187002 -2) (width 0.25) (layer B.Cu) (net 7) (status 20))
 (segment (start -66.187002 -2) (end -66.64 -2) (width 0.25) (layer B.Cu) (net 7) (status 30))
 (segment (start 5.72 -0.8) (end 3.257451 -3.262549) (width 0.25) (layer B.Cu) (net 7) (status 10))
 (segment (start -37.895 -2.130098) (end -36.762549 -3.262549) (width 0.09) (layer B.Cu) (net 7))
 (segment (start -37.895 0.6) (end -37.895 -2.130098) (width 0.09) (layer B.Cu) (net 7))
 (segment (start -36.762549 -3.262549) (end -64.924453 -3.262549) (width 0.25) (layer B.Cu) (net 7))
 (segment (start 3.257451 -3.262549) (end -36.762549 -3.262549) (width 0.25) (layer B.Cu) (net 7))
 (segment (start -64.1 -2) (end -61 -2) (width 0.25) (layer F.Cu) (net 8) (status 10))
 (segment (start -61 -2) (end -60.5 -2.5) (width 0.25) (layer F.Cu) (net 8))
 (segment (start -37.26 -0.581317) (end -37.26 -0.5) (width 0.25) (layer F.Cu) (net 8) (status 30))
 (segment (start -39.178683 -2.5) (end -37.26 -0.581317) (width 0.25) (layer F.Cu) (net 8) (status 20))
 (segment (start -60.5 -2.5) (end -39.178683 -2.5) (width 0.25) (layer F.Cu) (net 8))
 (segment (start -38.496135 -3.182548) (end -39.178683 -2.5) (width 0.25) (layer F.Cu) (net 8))
 (segment (start 4.517452 -3.182548) (end -38.496135 -3.182548) (width 0.25) (layer F.Cu) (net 8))
 (segment (start 6.809999 -0.890001) (end 4.517452 -3.182548) (width 0.25) (layer F.Cu) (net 8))
 (segment (start 6.809999 -0.159999) (end 6.809999 -0.890001) (width 0.25) (layer F.Cu) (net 8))
 (segment (start 6.35 0.3) (end 6.809999 -0.159999) (width 0.25) (layer F.Cu) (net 8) (status 10))
 (segment (start 4.45 0.6089) (end 4.45 -0.8) (width 0.135) (layer B.Cu) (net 9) (status 20))
 (segment (start -36.625 0.6) (end -34.217499 3.007501) (width 0.135) (layer B.Cu) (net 9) (status 10))
 (segment (start 2.033872 3.025028) (end 4.45 0.6089) (width 0.135) (layer B.Cu) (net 9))
 (segment (start -34.217499 3.007501) (end -34.199972 3.025028) (width 0.135) (layer B.Cu) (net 9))
 (segment (start -34.142471 3.082529) (end -34.217499 3.007501) (width 0.25) (layer B.Cu) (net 9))
 (segment (start 1.070902 3.082529) (end -34.142471 3.082529) (width 0.25) (layer B.Cu) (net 9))
 (segment (start 1.128403 3.025028) (end 1.070902 3.082529) (width 0.25) (layer B.Cu) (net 9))
 (segment (start 2.033872 3.025028) (end 1.128403 3.025028) (width 0.25) (layer B.Cu) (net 9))
 (segment (start -65.557471 3.082529) (end -66.64 2) (width 0.25) (layer B.Cu) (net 9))
 (segment (start -66.64 2) (end -65.24 3.4) (width 0.25) (layer B.Cu) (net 9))
 (segment (start -34.459942 3.4) (end -34.142471 3.082529) (width 0.25) (layer B.Cu) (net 9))
 (segment (start -65.24 3.4) (end -34.459942 3.4) (width 0.25) (layer B.Cu) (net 9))
 (segment (start -35.99 -0.5) (end -35.99 0.878902) (width 0.135) (layer F.Cu) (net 10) (status 10))
 (segment (start -35.99 0.878902) (end -33.863873 3.005029) (width 0.135) (layer F.Cu) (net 10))
 (segment (start -33.806372 3.06253) (end -33.863873 3.005029) (width 0.25) (layer F.Cu) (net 10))
 (segment (start 5.08 0.3) (end 2.31747 3.06253) (width 0.25) (layer F.Cu) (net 10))
 (segment (start -64.1 2) (end -62.7 3.4) (width 0.25) (layer F.Cu) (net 10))
 (segment (start -32.16253 3.06253) (end -33.806372 3.06253) (width 0.25) (layer F.Cu) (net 10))
 (segment (start 2.31747 3.06253) (end -32.16253 3.06253) (width 0.25) (layer F.Cu) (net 10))
 (segment (start -33.806372 3.06253) (end -34.16253 3.06253) (width 0.25) (layer F.Cu) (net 10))
 (segment (start -34.5 3.4) (end -62.7 3.4) (width 0.25) (layer F.Cu) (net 10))
 (segment (start -34.16253 3.06253) (end -34.5 3.4) (width 0.25) (layer F.Cu) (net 10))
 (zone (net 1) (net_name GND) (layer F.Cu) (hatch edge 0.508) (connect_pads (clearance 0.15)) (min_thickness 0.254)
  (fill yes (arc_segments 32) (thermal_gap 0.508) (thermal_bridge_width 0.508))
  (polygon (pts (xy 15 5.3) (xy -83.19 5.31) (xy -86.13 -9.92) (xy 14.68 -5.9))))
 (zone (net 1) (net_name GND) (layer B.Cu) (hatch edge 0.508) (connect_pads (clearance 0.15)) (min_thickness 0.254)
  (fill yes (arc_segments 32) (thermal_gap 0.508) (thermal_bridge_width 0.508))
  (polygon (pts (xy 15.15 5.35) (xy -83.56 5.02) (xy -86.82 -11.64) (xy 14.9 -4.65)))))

